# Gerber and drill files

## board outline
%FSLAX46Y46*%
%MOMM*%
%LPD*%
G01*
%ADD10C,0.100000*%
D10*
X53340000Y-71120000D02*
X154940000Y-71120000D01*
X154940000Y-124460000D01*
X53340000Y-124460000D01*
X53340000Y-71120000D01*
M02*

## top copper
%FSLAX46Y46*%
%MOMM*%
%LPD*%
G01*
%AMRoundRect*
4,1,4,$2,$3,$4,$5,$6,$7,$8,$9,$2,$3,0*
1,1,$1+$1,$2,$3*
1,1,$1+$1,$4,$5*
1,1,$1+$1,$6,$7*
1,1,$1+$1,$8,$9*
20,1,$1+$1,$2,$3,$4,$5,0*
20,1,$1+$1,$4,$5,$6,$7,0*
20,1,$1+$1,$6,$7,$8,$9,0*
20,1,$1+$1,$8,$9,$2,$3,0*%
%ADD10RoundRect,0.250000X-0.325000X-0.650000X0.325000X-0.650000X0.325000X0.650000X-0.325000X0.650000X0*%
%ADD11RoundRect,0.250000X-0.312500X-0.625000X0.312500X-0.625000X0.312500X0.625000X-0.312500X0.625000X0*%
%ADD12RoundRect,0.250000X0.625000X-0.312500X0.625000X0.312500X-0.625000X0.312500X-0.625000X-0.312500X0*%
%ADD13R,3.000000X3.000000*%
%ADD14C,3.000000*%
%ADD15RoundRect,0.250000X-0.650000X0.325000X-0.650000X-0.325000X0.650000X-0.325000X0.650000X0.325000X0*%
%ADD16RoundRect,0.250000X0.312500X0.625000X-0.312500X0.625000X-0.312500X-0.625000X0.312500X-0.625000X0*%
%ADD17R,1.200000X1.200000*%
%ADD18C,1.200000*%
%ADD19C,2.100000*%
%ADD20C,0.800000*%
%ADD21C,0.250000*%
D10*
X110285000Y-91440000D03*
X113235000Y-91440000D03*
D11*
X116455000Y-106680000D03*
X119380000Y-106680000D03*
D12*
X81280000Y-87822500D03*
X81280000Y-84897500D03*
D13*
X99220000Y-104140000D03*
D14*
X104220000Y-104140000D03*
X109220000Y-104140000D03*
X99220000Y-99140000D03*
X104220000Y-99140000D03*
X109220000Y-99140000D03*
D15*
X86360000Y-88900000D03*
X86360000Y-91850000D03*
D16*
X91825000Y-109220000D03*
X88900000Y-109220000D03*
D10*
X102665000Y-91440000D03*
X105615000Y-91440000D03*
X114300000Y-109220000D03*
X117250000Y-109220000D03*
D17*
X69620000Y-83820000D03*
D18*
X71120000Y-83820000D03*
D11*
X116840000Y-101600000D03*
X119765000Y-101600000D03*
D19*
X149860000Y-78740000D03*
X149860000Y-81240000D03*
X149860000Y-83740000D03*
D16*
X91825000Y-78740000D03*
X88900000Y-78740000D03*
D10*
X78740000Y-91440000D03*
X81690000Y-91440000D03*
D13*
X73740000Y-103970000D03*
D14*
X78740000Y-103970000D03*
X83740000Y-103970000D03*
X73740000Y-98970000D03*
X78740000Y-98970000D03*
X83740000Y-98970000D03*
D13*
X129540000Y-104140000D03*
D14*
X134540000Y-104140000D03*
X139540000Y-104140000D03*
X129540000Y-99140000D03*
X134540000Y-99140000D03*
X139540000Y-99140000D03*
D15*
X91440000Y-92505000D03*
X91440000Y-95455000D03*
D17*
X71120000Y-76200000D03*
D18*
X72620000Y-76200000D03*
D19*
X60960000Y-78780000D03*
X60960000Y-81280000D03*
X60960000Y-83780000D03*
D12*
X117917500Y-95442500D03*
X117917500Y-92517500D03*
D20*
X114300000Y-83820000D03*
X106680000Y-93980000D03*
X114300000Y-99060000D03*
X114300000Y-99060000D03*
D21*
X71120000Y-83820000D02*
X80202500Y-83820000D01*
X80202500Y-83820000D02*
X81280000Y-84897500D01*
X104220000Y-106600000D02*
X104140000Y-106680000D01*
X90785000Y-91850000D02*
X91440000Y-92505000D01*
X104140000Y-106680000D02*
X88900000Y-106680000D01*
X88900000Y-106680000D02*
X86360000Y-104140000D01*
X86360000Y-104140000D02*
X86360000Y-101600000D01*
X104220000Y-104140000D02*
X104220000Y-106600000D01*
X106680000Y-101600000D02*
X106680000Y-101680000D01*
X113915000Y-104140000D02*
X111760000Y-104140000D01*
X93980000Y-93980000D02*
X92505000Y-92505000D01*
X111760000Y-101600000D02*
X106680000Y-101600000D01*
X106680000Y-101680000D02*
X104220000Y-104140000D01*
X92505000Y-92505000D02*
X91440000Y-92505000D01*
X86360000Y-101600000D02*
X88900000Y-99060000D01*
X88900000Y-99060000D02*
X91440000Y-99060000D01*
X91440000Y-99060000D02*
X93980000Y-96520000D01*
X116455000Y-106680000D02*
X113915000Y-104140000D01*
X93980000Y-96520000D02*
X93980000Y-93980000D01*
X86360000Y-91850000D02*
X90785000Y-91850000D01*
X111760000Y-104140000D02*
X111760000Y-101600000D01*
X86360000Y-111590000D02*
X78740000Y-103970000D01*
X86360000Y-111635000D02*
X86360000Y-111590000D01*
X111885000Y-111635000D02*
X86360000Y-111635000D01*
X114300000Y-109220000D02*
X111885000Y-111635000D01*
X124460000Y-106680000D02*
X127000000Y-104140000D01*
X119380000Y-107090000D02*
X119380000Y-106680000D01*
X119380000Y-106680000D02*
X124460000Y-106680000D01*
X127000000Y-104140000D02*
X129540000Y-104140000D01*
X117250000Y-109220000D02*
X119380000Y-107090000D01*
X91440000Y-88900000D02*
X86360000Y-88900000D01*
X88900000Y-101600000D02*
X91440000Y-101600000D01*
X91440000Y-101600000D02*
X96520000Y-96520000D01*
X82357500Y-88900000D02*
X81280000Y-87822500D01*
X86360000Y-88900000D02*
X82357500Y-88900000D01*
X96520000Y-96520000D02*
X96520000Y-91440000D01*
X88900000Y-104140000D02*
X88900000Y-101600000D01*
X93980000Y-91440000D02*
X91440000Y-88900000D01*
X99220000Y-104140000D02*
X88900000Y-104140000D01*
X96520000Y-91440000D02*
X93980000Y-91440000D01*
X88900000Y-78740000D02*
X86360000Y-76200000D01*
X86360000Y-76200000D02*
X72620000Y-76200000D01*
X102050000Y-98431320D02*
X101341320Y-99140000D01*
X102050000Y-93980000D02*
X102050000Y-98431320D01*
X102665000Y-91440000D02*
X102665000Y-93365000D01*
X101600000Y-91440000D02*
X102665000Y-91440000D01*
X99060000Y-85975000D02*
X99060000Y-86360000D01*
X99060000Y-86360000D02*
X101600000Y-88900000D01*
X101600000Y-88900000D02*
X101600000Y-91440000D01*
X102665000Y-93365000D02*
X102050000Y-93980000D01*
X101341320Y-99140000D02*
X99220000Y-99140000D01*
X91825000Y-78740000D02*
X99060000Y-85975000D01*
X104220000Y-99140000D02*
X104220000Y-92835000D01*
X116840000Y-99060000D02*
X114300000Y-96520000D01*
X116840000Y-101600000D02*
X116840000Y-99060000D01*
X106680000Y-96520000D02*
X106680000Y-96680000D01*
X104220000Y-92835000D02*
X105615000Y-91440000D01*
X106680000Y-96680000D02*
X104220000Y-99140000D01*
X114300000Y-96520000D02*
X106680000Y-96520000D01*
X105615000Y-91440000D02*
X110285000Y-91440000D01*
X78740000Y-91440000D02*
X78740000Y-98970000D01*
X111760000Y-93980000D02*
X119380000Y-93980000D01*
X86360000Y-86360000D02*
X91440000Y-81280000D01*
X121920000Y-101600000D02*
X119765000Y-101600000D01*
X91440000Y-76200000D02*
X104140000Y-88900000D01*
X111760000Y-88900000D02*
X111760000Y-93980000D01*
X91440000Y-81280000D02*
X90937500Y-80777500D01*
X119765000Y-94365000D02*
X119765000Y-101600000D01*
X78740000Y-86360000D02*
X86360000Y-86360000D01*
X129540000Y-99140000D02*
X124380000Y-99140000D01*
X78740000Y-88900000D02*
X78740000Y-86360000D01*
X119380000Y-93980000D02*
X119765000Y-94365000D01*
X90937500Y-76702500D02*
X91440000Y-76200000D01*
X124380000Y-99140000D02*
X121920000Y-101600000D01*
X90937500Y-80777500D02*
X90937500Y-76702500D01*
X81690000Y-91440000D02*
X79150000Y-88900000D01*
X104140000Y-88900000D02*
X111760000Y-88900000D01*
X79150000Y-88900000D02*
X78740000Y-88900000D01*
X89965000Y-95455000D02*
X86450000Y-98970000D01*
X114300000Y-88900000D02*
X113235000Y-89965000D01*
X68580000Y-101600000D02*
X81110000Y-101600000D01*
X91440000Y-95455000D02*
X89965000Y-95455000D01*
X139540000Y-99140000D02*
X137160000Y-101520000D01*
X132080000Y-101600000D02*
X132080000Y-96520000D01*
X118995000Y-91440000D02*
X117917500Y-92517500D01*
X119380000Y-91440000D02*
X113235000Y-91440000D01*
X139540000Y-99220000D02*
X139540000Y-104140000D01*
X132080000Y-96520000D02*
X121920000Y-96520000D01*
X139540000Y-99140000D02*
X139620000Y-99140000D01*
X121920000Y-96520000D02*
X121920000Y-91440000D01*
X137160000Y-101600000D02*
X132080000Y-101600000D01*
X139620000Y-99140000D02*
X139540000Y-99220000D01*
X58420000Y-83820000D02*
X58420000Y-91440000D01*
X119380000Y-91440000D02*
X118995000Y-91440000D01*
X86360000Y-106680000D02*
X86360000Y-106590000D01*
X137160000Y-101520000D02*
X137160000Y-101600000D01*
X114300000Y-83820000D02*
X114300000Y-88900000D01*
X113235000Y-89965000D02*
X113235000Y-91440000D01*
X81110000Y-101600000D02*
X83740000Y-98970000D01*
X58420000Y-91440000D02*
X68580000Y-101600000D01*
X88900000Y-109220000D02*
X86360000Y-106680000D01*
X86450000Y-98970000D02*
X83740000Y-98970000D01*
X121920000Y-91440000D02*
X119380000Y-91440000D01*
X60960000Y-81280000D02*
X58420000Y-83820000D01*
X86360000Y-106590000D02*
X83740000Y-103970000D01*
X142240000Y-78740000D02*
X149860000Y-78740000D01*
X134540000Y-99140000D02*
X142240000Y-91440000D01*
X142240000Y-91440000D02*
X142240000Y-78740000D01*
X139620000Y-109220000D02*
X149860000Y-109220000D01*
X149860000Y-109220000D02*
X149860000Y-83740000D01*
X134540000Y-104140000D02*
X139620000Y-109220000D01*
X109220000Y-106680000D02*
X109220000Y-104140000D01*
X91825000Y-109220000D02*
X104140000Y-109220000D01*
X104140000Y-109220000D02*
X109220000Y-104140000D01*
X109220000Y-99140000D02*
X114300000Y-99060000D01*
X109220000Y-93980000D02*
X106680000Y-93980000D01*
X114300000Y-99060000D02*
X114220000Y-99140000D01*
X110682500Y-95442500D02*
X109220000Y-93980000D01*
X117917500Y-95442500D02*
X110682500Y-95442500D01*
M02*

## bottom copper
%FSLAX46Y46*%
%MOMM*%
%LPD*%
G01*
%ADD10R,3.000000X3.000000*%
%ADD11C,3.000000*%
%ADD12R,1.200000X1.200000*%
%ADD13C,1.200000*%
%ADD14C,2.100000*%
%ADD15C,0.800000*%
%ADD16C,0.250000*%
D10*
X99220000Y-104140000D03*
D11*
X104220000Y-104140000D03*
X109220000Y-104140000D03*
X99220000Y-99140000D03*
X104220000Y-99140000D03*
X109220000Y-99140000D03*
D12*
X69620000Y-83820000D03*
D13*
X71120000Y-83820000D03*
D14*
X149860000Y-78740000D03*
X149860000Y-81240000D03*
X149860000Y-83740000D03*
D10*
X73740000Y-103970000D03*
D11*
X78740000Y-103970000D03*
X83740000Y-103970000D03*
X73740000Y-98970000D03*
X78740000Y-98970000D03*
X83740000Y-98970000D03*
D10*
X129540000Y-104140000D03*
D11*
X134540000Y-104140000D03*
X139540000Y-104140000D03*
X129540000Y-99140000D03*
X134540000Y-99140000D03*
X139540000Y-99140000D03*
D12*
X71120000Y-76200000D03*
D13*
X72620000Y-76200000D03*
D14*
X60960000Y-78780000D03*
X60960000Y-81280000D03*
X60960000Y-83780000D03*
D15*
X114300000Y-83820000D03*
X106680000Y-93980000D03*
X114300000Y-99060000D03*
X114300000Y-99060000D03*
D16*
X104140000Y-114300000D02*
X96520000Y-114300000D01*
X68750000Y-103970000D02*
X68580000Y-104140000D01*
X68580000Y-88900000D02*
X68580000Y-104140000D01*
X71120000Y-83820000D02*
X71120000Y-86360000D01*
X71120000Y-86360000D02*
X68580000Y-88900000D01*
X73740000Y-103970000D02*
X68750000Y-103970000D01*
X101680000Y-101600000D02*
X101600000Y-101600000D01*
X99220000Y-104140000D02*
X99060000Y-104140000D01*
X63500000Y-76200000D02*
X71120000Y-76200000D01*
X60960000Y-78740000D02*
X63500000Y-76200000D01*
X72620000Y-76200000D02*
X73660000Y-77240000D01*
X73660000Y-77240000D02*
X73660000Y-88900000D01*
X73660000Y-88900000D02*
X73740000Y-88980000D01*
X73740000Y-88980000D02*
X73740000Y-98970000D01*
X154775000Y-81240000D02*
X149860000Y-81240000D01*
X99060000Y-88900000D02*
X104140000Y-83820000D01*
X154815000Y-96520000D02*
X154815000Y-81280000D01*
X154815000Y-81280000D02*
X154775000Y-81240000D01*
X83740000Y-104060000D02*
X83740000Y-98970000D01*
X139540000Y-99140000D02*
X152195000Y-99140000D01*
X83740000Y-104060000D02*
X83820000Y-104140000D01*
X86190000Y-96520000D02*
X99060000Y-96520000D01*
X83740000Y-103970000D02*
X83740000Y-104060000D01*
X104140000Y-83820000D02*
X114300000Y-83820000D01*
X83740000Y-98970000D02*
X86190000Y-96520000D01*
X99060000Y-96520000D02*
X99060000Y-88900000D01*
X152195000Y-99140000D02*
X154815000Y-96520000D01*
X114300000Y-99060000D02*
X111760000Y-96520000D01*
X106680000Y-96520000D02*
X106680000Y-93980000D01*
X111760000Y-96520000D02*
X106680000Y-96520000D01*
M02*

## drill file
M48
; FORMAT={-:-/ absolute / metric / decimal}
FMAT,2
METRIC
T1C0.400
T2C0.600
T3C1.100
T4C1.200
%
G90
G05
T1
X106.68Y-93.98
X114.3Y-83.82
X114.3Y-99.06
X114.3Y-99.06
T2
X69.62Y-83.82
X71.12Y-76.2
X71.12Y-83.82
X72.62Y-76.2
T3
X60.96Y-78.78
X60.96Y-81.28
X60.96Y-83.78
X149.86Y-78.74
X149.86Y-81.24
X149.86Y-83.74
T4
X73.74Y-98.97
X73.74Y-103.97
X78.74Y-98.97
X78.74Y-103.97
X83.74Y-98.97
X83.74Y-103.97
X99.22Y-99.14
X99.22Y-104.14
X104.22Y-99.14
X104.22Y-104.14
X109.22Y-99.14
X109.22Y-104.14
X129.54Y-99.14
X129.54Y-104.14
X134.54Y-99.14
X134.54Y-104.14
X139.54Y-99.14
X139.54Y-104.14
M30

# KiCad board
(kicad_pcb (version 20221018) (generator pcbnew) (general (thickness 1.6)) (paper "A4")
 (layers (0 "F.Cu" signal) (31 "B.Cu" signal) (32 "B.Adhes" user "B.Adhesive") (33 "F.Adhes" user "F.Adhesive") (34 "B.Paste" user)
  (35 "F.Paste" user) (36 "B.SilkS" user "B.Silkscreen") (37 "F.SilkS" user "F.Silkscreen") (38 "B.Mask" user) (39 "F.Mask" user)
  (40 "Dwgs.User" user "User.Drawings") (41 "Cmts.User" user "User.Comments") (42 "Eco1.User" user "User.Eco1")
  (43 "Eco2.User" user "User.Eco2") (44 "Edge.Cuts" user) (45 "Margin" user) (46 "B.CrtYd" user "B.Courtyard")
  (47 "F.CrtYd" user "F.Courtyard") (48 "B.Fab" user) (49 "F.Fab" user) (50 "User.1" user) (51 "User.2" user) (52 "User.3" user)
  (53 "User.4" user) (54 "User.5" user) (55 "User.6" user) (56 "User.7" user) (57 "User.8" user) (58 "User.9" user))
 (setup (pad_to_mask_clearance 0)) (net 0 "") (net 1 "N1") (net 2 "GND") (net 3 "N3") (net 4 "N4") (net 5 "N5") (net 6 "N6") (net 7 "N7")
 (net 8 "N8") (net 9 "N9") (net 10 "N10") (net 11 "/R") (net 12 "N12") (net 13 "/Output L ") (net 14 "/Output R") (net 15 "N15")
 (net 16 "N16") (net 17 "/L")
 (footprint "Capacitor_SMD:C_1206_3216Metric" (layer "F.Cu") (at 111.76 91.44)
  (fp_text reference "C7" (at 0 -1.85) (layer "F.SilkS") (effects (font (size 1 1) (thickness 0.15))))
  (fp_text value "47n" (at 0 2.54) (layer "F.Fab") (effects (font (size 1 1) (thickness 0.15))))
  (pad "1" smd roundrect (at -1.475 0) (size 1.15 1.8) (layers "F.Cu" "F.Paste" "F.Mask") (roundrect_rratio 0.217391) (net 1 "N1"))
  (pad "2" smd roundrect (at 1.475 0) (size 1.15 1.8) (layers "F.Cu" "F.Paste" "F.Mask") (roundrect_rratio 0.217391) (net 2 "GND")))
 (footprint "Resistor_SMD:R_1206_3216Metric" (layer "F.Cu") (at 117.9175 106.68)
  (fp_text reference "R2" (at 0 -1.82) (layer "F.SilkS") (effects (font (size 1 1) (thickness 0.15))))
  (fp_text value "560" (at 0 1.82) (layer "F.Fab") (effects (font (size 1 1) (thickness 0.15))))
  (pad "1" smd roundrect (at -1.4625 0) (size 1.125 1.75) (layers "F.Cu" "F.Paste" "F.Mask") (roundrect_rratio 0.222222) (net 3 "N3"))
  (pad "2" smd roundrect (at 1.4625 0) (size 1.125 1.75) (layers "F.Cu" "F.Paste" "F.Mask") (roundrect_rratio 0.222222) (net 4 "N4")))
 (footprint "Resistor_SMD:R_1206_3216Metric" (layer "F.Cu") (at 81.28 86.36 90)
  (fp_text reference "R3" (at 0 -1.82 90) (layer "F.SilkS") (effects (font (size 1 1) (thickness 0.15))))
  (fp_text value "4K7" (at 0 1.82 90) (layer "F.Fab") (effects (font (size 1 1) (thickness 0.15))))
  (pad "1" smd roundrect (at -1.4625 0 90) (size 1.125 1.75) (layers "F.Cu" "F.Paste" "F.Mask") (roundrect_rratio 0.222222) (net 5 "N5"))
  (pad "2" smd roundrect (at 1.4625 0 90) (size 1.125 1.75) (layers "F.Cu" "F.Paste" "F.Mask") (roundrect_rratio 0.222222) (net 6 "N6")))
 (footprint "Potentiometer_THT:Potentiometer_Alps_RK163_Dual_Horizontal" (layer "F.Cu") (at 99.22 104.14 90)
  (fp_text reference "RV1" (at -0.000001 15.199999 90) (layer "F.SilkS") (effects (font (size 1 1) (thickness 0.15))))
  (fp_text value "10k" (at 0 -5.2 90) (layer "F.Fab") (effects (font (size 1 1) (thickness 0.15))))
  (pad "1" thru_hole rect (at 0 0 270) (size 3 3) (drill 1.2) (layers "*.Cu" "*.Mask") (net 5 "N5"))
  (pad "2" thru_hole circle (at 0 5 270) (size 3 3) (drill 1.2) (layers "*.Cu" "*.Mask") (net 3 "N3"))
  (pad "3" thru_hole circle (at 0 10 270) (size 3 3) (drill 1.2) (layers "*.Cu" "*.Mask") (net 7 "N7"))
  (pad "4" thru_hole circle (at 5 0 270) (size 3 3) (drill 1.2) (layers "*.Cu" "*.Mask") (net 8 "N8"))
  (pad "5" thru_hole circle (at 5 5 270) (size 3 3) (drill 1.2) (layers "*.Cu" "*.Mask") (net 1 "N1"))
  (pad "6" thru_hole circle (at 5 10 270) (size 3 3) (drill 1.2) (layers "*.Cu" "*.Mask") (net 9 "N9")))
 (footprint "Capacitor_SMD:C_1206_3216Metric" (layer "F.Cu") (at 86.36 90.375 -90)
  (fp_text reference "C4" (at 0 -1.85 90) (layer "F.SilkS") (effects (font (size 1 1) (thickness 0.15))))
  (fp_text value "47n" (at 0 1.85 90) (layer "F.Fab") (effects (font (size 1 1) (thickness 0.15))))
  (pad "1" smd roundrect (at -1.475 0 270) (size 1.15 1.8) (layers "F.Cu" "F.Paste" "F.Mask") (roundrect_rratio 0.217391) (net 5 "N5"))
  (pad "2" smd roundrect (at 1.475 0 270) (size 1.15 1.8) (layers "F.Cu" "F.Paste" "F.Mask") (roundrect_rratio 0.217391) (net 3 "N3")))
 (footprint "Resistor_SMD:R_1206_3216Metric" (layer "F.Cu") (at 90.3625 109.22 180)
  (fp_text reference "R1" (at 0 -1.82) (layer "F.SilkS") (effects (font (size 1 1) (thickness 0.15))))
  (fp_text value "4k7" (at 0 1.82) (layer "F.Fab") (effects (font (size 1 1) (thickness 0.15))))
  (pad "1" smd roundrect (at -1.4625 0 180) (size 1.125 1.75) (layers "F.Cu" "F.Paste" "F.Mask") (roundrect_rratio 0.222222) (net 7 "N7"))
  (pad "2" smd roundrect (at 1.4625 0 180) (size 1.125 1.75) (layers "F.Cu" "F.Paste" "F.Mask") (roundrect_rratio 0.222222) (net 2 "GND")))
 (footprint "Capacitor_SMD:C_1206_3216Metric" (layer "F.Cu") (at 104.14 91.44)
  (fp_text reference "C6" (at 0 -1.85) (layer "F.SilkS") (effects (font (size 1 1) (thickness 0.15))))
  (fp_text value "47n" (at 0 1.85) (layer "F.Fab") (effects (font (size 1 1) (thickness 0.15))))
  (pad "1" smd roundrect (at -1.475 0) (size 1.15 1.8) (layers "F.Cu" "F.Paste" "F.Mask") (roundrect_rratio 0.217391) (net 8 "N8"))
  (pad "2" smd roundrect (at 1.475 0) (size 1.15 1.8) (layers "F.Cu" "F.Paste" "F.Mask") (roundrect_rratio 0.217391) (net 1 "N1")))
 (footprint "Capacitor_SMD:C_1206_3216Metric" (layer "F.Cu") (at 115.775 109.22)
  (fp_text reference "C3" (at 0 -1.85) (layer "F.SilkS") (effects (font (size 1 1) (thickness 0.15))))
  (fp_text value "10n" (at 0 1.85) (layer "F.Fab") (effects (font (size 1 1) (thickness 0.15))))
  (pad "1" smd roundrect (at -1.475 0) (size 1.15 1.8) (layers "F.Cu" "F.Paste" "F.Mask") (roundrect_rratio 0.217391) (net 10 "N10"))
  (pad "2" smd roundrect (at 1.475 0) (size 1.15 1.8) (layers "F.Cu" "F.Paste" "F.Mask") (roundrect_rratio 0.217391) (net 4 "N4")))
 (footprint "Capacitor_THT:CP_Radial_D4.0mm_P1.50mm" (layer "F.Cu") (at 69.62 83.82)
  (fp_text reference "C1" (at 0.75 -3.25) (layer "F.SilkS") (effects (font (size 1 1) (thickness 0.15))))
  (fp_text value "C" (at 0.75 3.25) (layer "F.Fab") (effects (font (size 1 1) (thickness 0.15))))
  (pad "1" thru_hole rect (at 0 0) (size 1.2 1.2) (drill 0.6) (layers "*.Cu" "*.Mask") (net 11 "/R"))
  (pad "2" thru_hole circle (at 1.5 0) (size 1.2 1.2) (drill 0.6) (layers "*.Cu" "*.Mask") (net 6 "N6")))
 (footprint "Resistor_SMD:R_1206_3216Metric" (layer "F.Cu") (at 118.3025 101.6)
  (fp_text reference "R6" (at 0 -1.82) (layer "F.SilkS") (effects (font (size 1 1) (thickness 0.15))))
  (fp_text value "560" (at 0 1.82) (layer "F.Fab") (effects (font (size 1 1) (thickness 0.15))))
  (pad "1" smd roundrect (at -1.4625 0) (size 1.125 1.75) (layers "F.Cu" "F.Paste" "F.Mask") (roundrect_rratio 0.222222) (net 1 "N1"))
  (pad "2" smd roundrect (at 1.4625 0) (size 1.125 1.75) (layers "F.Cu" "F.Paste" "F.Mask") (roundrect_rratio 0.222222) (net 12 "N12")))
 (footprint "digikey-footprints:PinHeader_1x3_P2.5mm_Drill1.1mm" (layer "F.Cu") (at 149.86 78.74 -90)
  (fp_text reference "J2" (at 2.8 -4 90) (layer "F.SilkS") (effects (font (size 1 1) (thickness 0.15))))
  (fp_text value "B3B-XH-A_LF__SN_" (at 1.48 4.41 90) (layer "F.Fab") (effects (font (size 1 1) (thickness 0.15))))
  (pad "1" thru_hole circle (at 0 0 270) (size 2.1 2.1) (drill 1.1) (layers "*.Cu" "*.Mask") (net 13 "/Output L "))
  (pad "2" thru_hole circle (at 2.5 0 270) (size 2.1 2.1) (drill 1.1) (layers "*.Cu" "*.Mask") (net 2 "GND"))
  (pad "3" thru_hole circle (at 5 0 270) (size 2.1 2.1) (drill 1.1) (layers "*.Cu" "*.Mask") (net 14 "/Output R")))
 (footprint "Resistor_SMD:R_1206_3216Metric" (layer "F.Cu") (at 90.3625 78.74 180)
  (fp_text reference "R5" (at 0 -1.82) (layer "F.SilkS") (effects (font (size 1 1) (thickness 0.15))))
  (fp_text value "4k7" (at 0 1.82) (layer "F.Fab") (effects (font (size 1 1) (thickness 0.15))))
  (pad "1" smd roundrect (at -1.4625 0 180) (size 1.125 1.75) (layers "F.Cu" "F.Paste" "F.Mask") (roundrect_rratio 0.222222) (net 8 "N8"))
  (pad "2" smd roundrect (at 1.4625 0 180) (size 1.125 1.75) (layers "F.Cu" "F.Paste" "F.Mask") (roundrect_rratio 0.222222) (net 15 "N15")))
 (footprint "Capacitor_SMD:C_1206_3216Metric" (layer "F.Cu") (at 80.215 91.44)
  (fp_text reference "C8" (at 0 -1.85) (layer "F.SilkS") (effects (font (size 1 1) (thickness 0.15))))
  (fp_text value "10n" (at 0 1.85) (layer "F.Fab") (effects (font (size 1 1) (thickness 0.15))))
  (pad "1" smd roundrect (at -1.475 0) (size 1.15 1.8) (layers "F.Cu" "F.Paste" "F.Mask") (roundrect_rratio 0.217391) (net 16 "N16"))
  (pad "2" smd roundrect (at 1.475 0) (size 1.15 1.8) (layers "F.Cu" "F.Paste" "F.Mask") (roundrect_rratio 0.217391) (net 12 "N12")))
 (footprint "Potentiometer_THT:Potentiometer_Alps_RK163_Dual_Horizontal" (layer "F.Cu") (at 73.74 103.97 90)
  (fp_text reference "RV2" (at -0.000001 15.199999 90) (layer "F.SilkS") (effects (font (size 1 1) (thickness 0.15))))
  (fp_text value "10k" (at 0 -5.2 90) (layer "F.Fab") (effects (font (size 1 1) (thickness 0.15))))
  (pad "1" thru_hole rect (at 0 0 270) (size 3 3) (drill 1.2) (layers "*.Cu" "*.Mask") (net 6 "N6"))
  (pad "2" thru_hole circle (at 0 5 270) (size 3 3) (drill 1.2) (layers "*.Cu" "*.Mask") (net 10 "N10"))
  (pad "3" thru_hole circle (at 0 10 270) (size 3 3) (drill 1.2) (layers "*.Cu" "*.Mask") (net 2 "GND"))
  (pad "4" thru_hole circle (at 5 0 270) (size 3 3) (drill 1.2) (layers "*.Cu" "*.Mask") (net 15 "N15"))
  (pad "5" thru_hole circle (at 5 5 270) (size 3 3) (drill 1.2) (layers "*.Cu" "*.Mask") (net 16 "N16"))
  (pad "6" thru_hole circle (at 5 10 270) (size 3 3) (drill 1.2) (layers "*.Cu" "*.Mask") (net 2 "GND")))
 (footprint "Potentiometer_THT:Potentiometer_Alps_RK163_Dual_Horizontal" (layer "F.Cu") (at 129.54 104.14 90)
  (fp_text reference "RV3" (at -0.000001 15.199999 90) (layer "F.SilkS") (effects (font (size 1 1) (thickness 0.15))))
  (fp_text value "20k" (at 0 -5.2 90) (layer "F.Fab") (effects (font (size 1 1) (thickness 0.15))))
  (pad "1" thru_hole rect (at 0 0 270) (size 3 3) (drill 1.2) (layers "*.Cu" "*.Mask") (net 4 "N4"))
  (pad "2" thru_hole circle (at 0 5 270) (size 3 3) (drill 1.2) (layers "*.Cu" "*.Mask") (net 14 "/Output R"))
  (pad "3" thru_hole circle (at 0 10 270) (size 3 3) (drill 1.2) (layers "*.Cu" "*.Mask") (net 2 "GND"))
  (pad "4" thru_hole circle (at 5 0 270) (size 3 3) (drill 1.2) (layers "*.Cu" "*.Mask") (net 12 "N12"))
  (pad "5" thru_hole circle (at 5 5 270) (size 3 3) (drill 1.2) (layers "*.Cu" "*.Mask") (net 13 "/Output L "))
  (pad "6" thru_hole circle (at 5 10 270) (size 3 3) (drill 1.2) (layers "*.Cu" "*.Mask") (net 2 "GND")))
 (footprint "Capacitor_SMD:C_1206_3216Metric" (layer "F.Cu") (at 91.44 93.98 -90)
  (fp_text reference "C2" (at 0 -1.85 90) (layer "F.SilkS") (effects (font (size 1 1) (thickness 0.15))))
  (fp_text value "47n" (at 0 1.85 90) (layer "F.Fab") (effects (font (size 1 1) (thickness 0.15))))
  (pad "1" smd roundrect (at -1.475 0 270) (size 1.15 1.8) (layers "F.Cu" "F.Paste" "F.Mask") (roundrect_rratio 0.217391) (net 3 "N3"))
  (pad "2" smd roundrect (at 1.475 0 270) (size 1.15 1.8) (layers "F.Cu" "F.Paste" "F.Mask") (roundrect_rratio 0.217391) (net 2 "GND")))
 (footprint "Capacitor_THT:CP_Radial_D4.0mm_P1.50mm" (layer "F.Cu") (at 71.12 76.2)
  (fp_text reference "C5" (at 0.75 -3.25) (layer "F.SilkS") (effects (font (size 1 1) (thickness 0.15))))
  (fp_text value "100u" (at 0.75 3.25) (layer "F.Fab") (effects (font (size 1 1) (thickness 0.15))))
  (pad "1" thru_hole rect (at 0 0) (size 1.2 1.2) (drill 0.6) (layers "*.Cu" "*.Mask") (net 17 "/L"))
  (pad "2" thru_hole circle (at 1.5 0) (size 1.2 1.2) (drill 0.6) (layers "*.Cu" "*.Mask") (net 15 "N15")))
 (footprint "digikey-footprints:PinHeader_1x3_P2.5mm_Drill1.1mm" (layer "F.Cu") (at 60.96 78.78 -90)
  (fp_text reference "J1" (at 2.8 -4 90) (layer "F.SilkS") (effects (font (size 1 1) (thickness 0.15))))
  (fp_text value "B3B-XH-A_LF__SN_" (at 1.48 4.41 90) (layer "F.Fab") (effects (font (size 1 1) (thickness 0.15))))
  (pad "1" thru_hole circle (at 0 0 270) (size 2.1 2.1) (drill 1.1) (layers "*.Cu" "*.Mask") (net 17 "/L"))
  (pad "2" thru_hole circle (at 2.5 0 270) (size 2.1 2.1) (drill 1.1) (layers "*.Cu" "*.Mask") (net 2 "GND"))
  (pad "3" thru_hole circle (at 5 0 270) (size 2.1 2.1) (drill 1.1) (layers "*.Cu" "*.Mask") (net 11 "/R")))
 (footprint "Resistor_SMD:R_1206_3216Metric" (layer "F.Cu") (at 117.9175 93.98 90)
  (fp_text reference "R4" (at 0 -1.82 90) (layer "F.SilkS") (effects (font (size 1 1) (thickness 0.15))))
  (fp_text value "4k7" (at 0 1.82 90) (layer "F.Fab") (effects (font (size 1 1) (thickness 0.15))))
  (pad "1" smd roundrect (at -1.4625 0 90) (size 1.125 1.75) (layers "F.Cu" "F.Paste" "F.Mask") (roundrect_rratio 0.222222) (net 9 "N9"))
  (pad "2" smd roundrect (at 1.4625 0 90) (size 1.125 1.75) (layers "F.Cu" "F.Paste" "F.Mask") (roundrect_rratio 0.222222) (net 2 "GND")))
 (gr_rect (start 53.34 71.12) (end 154.94 124.46) (stroke (width 0.1) (type default)) (fill none) (layer "Edge.Cuts"))
 (segment (start 104.14 114.3) (end 96.52 114.3) (width 0.25) (layer "B.Cu") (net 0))
 (segment (start 71.12 83.82) (end 80.2025 83.82) (width 0.25) (layer "F.Cu") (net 6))
 (segment (start 80.2025 83.82) (end 81.28 84.8975) (width 0.25) (layer "F.Cu") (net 6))
 (segment (start 68.75 103.97) (end 68.58 104.14) (width 0.25) (layer "B.Cu") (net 6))
 (segment (start 68.58 88.9) (end 68.58 104.14) (width 0.25) (layer "B.Cu") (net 6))
 (segment (start 71.12 83.82) (end 71.12 86.36) (width 0.25) (layer "B.Cu") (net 6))
 (segment (start 71.12 86.36) (end 68.58 88.9) (width 0.25) (layer "B.Cu") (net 6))
 (segment (start 73.74 103.97) (end 68.75 103.97) (width 0.25) (layer "B.Cu") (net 6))
 (segment (start 104.22 106.6) (end 104.14 106.68) (width 0.25) (layer "F.Cu") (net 3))
 (segment (start 90.785 91.85) (end 91.44 92.505) (width 0.25) (layer "F.Cu") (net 3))
 (segment (start 104.14 106.68) (end 88.9 106.68) (width 0.25) (layer "F.Cu") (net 3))
 (segment (start 88.9 106.68) (end 86.36 104.14) (width 0.25) (layer "F.Cu") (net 3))
 (segment (start 86.36 104.14) (end 86.36 101.6) (width 0.25) (layer "F.Cu") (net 3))
 (segment (start 104.22 104.14) (end 104.22 106.6) (width 0.25) (layer "F.Cu") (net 3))
 (segment (start 106.68 101.6) (end 106.68 101.68) (width 0.25) (layer "F.Cu") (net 3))
 (segment (start 113.915 104.14) (end 111.76 104.14) (width 0.25) (layer "F.Cu") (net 3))
 (segment (start 93.98 93.98) (end 92.505 92.505) (width 0.25) (layer "F.Cu") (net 3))
 (segment (start 111.76 101.6) (end 106.68 101.6) (width 0.25) (layer "F.Cu") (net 3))
 (segment (start 106.68 101.68) (end 104.22 104.14) (width 0.25) (layer "F.Cu") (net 3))
 (segment (start 92.505 92.505) (end 91.44 92.505) (width 0.25) (layer "F.Cu") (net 3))
 (segment (start 86.36 101.6) (end 88.9 99.06) (width 0.25) (layer "F.Cu") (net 3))
 (segment (start 88.9 99.06) (end 91.44 99.06) (width 0.25) (layer "F.Cu") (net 3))
 (segment (start 91.44 99.06) (end 93.98 96.52) (width 0.25) (layer "F.Cu") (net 3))
 (segment (start 116.455 106.68) (end 113.915 104.14) (width 0.25) (layer "F.Cu") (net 3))
 (segment (start 93.98 96.52) (end 93.98 93.98) (width 0.25) (layer "F.Cu") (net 3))
 (segment (start 86.36 91.85) (end 90.785 91.85) (width 0.25) (layer "F.Cu") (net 3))
 (segment (start 111.76 104.14) (end 111.76 101.6) (width 0.25) (layer "F.Cu") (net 3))
 (segment (start 101.68 101.6) (end 101.6 101.6) (width 0.25) (layer "B.Cu") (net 3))
 (segment (start 86.36 111.59) (end 78.74 103.97) (width 0.25) (layer "F.Cu") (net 10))
 (segment (start 86.36 111.635) (end 86.36 111.59) (width 0.25) (layer "F.Cu") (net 10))
 (segment (start 111.885 111.635) (end 86.36 111.635) (width 0.25) (layer "F.Cu") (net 10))
 (segment (start 114.3 109.22) (end 111.885 111.635) (width 0.25) (layer "F.Cu") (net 10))
 (segment (start 124.46 106.68) (end 127 104.14) (width 0.25) (layer "F.Cu") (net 4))
 (segment (start 119.38 107.09) (end 119.38 106.68) (width 0.25) (layer "F.Cu") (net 4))
 (segment (start 119.38 106.68) (end 124.46 106.68) (width 0.25) (layer "F.Cu") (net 4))
 (segment (start 127 104.14) (end 129.54 104.14) (width 0.25) (layer "F.Cu") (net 4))
 (segment (start 117.25 109.22) (end 119.38 107.09) (width 0.25) (layer "F.Cu") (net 4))
 (segment (start 91.44 88.9) (end 86.36 88.9) (width 0.25) (layer "F.Cu") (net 5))
 (segment (start 88.9 101.6) (end 91.44 101.6) (width 0.25) (layer "F.Cu") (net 5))
 (segment (start 91.44 101.6) (end 96.52 96.52) (width 0.25) (layer "F.Cu") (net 5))
 (segment (start 82.3575 88.9) (end 81.28 87.8225) (width 0.25) (layer "F.Cu") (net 5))
 (segment (start 86.36 88.9) (end 82.3575 88.9) (width 0.25) (layer "F.Cu") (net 5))
 (segment (start 96.52 96.52) (end 96.52 91.44) (width 0.25) (layer "F.Cu") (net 5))
 (segment (start 88.9 104.14) (end 88.9 101.6) (width 0.25) (layer "F.Cu") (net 5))
 (segment (start 93.98 91.44) (end 91.44 88.9) (width 0.25) (layer "F.Cu") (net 5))
 (segment (start 99.22 104.14) (end 88.9 104.14) (width 0.25) (layer "F.Cu") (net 5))
 (segment (start 96.52 91.44) (end 93.98 91.44) (width 0.25) (layer "F.Cu") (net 5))
 (segment (start 99.22 104.14) (end 99.06 104.14) (width 0.25) (layer "B.Cu") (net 5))
 (segment (start 63.5 76.2) (end 71.12 76.2) (width 0.25) (layer "B.Cu") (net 17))
 (segment (start 60.96 78.74) (end 63.5 76.2) (width 0.25) (layer "B.Cu") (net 17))
 (segment (start 88.9 78.74) (end 86.36 76.2) (width 0.25) (layer "F.Cu") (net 15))
 (segment (start 86.36 76.2) (end 72.62 76.2) (width 0.25) (layer "F.Cu") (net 15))
 (segment (start 72.62 76.2) (end 73.66 77.24) (width 0.25) (layer "B.Cu") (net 15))
 (segment (start 73.66 77.24) (end 73.66 88.9) (width 0.25) (layer "B.Cu") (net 15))
 (segment (start 73.66 88.9) (end 73.74 88.98) (width 0.25) (layer "B.Cu") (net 15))
 (segment (start 73.74 88.98) (end 73.74 98.97) (width 0.25) (layer "B.Cu") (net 15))
 (segment (start 102.05 98.43132) (end 101.34132 99.14) (width 0.25) (layer "F.Cu") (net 8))
 (segment (start 102.05 93.98) (end 102.05 98.43132) (width 0.25) (layer "F.Cu") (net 8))
 (segment (start 102.665 91.44) (end 102.665 93.365) (width 0.25) (layer "F.Cu") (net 8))
 (segment (start 101.6 91.44) (end 102.665 91.44) (width 0.25) (layer "F.Cu") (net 8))
 (segment (start 99.06 85.975) (end 99.06 86.36) (width 0.25) (layer "F.Cu") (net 8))
 (segment (start 99.06 86.36) (end 101.6 88.9) (width 0.25) (layer "F.Cu") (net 8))
 (segment (start 101.6 88.9) (end 101.6 91.44) (width 0.25) (layer "F.Cu") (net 8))
 (segment (start 102.665 93.365) (end 102.05 93.98) (width 0.25) (layer "F.Cu") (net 8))
 (segment (start 101.34132 99.14) (end 99.22 99.14) (width 0.25) (layer "F.Cu") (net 8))
 (segment (start 91.825 78.74) (end 99.06 85.975) (width 0.25) (layer "F.Cu") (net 8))
 (segment (start 104.22 99.14) (end 104.22 92.835) (width 0.25) (layer "F.Cu") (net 1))
 (segment (start 116.84 99.06) (end 114.3 96.52) (width 0.25) (layer "F.Cu") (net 1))
 (segment (start 116.84 101.6) (end 116.84 99.06) (width 0.25) (layer "F.Cu") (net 1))
 (segment (start 106.68 96.52) (end 106.68 96.68) (width 0.25) (layer "F.Cu") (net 1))
 (segment (start 104.22 92.835) (end 105.615 91.44) (width 0.25) (layer "F.Cu") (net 1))
 (segment (start 106.68 96.68) (end 104.22 99.14) (width 0.25) (layer "F.Cu") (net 1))
 (segment (start 114.3 96.52) (end 106.68 96.52) (width 0.25) (layer "F.Cu") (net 1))
 (segment (start 105.615 91.44) (end 110.285 91.44) (width 0.25) (layer "F.Cu") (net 1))
 (segment (start 78.74 91.44) (end 78.74 98.97) (width 0.25) (layer "F.Cu") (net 16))
 (segment (start 111.76 93.98) (end 119.38 93.98) (width 0.25) (layer "F.Cu") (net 12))
 (segment (start 86.36 86.36) (end 91.44 81.28) (width 0.25) (layer "F.Cu") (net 12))
 (segment (start 121.92 101.6) (end 119.765 101.6) (width 0.25) (layer "F.Cu") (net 12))
 (segment (start 91.44 76.2) (end 104.14 88.9) (width 0.25) (layer "F.Cu") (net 12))
 (segment (start 111.76 88.9) (end 111.76 93.98) (width 0.25) (layer "F.Cu") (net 12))
 (segment (start 91.44 81.28) (end 90.9375 80.7775) (width 0.25) (layer "F.Cu") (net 12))
 (segment (start 119.765 94.365) (end 119.765 101.6) (width 0.25) (layer "F.Cu") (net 12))
 (segment (start 78.74 86.36) (end 86.36 86.36) (width 0.25) (layer "F.Cu") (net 12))
 (segment (start 129.54 99.14) (end 124.38 99.14) (width 0.25) (layer "F.Cu") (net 12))
 (segment (start 78.74 88.9) (end 78.74 86.36) (width 0.25) (layer "F.Cu") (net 12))
 (segment (start 119.38 93.98) (end 119.765 94.365) (width 0.25) (layer "F.Cu") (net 12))
 (segment (start 90.9375 76.7025) (end 91.44 76.2) (width 0.25) (layer "F.Cu") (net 12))
 (segment (start 124.38 99.14) (end 121.92 101.6) (width 0.25) (layer "F.Cu") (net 12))
 (segment (start 90.9375 80.7775) (end 90.9375 76.7025) (width 0.25) (layer "F.Cu") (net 12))
 (segment (start 81.69 91.44) (end 79.15 88.9) (width 0.25) (layer "F.Cu") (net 12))
 (segment (start 104.14 88.9) (end 111.76 88.9) (width 0.25) (layer "F.Cu") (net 12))
 (segment (start 79.15 88.9) (end 78.74 88.9) (width 0.25) (layer "F.Cu") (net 12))
 (segment (start 89.965 95.455) (end 86.45 98.97) (width 0.25) (layer "F.Cu") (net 2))
 (segment (start 114.3 88.9) (end 113.235 89.965) (width 0.25) (layer "F.Cu") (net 2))
 (segment (start 68.58 101.6) (end 81.11 101.6) (width 0.25) (layer "F.Cu") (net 2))
 (segment (start 91.44 95.455) (end 89.965 95.455) (width 0.25) (layer "F.Cu") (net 2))
 (segment (start 139.54 99.14) (end 137.16 101.52) (width 0.25) (layer "F.Cu") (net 2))
 (segment (start 132.08 101.6) (end 132.08 96.52) (width 0.25) (layer "F.Cu") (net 2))
 (segment (start 118.995 91.44) (end 117.9175 92.5175) (width 0.25) (layer "F.Cu") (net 2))
 (segment (start 119.38 91.44) (end 113.235 91.44) (width 0.25) (layer "F.Cu") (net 2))
 (segment (start 139.54 99.22) (end 139.54 104.14) (width 0.25) (layer "F.Cu") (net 2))
 (segment (start 132.08 96.52) (end 121.92 96.52) (width 0.25) (layer "F.Cu") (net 2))
 (segment (start 139.54 99.14) (end 139.62 99.14) (width 0.25) (layer "F.Cu") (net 2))
 (segment (start 121.92 96.52) (end 121.92 91.44) (width 0.25) (layer "F.Cu") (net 2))
 (segment (start 137.16 101.6) (end 132.08 101.6) (width 0.25) (layer "F.Cu") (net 2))
 (segment (start 139.62 99.14) (end 139.54 99.22) (width 0.25) (layer "F.Cu") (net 2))
 (segment (start 58.42 83.82) (end 58.42 91.44) (width 0.25) (layer "F.Cu") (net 2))
 (segment (start 119.38 91.44) (end 118.995 91.44) (width 0.25) (layer "F.Cu") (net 2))
 (segment (start 86.36 106.68) (end 86.36 106.59) (width 0.25) (layer "F.Cu") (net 2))
 (segment (start 137.16 101.52) (end 137.16 101.6) (width 0.25) (layer "F.Cu") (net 2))
 (segment (start 114.3 83.82) (end 114.3 88.9) (width 0.25) (layer "F.Cu") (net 2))
 (segment (start 113.235 89.965) (end 113.235 91.44) (width 0.25) (layer "F.Cu") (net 2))
 (segment (start 81.11 101.6) (end 83.74 98.97) (width 0.25) (layer "F.Cu") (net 2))
 (segment (start 58.42 91.44) (end 68.58 101.6) (width 0.25) (layer "F.Cu") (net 2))
 (segment (start 88.9 109.22) (end 86.36 106.68) (width 0.25) (layer "F.Cu") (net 2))
 (segment (start 86.45 98.97) (end 83.74 98.97) (width 0.25) (layer "F.Cu") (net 2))
 (segment (start 121.92 91.44) (end 119.38 91.44) (width 0.25) (layer "F.Cu") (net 2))
 (segment (start 60.96 81.28) (end 58.42 83.82) (width 0.25) (layer "F.Cu") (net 2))
 (segment (start 86.36 106.59) (end 83.74 103.97) (width 0.25) (layer "F.Cu") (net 2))
 (via (at 114.3 83.82) (size 0.8) (drill 0.4) (layers "F.Cu" "B.Cu") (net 2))
 (segment (start 154.775 81.24) (end 149.86 81.24) (width 0.25) (layer "B.Cu") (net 2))
 (segment (start 99.06 88.9) (end 104.14 83.82) (width 0.25) (layer "B.Cu") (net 2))
 (segment (start 154.815 96.52) (end 154.815 81.28) (width 0.25) (layer "B.Cu") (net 2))
 (segment (start 154.815 81.28) (end 154.775 81.24) (width 0.25) (layer "B.Cu") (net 2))
 (segment (start 83.74 104.06) (end 83.74 98.97) (width 0.25) (layer "B.Cu") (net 2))
 (segment (start 139.54 99.14) (end 152.195 99.14) (width 0.25) (layer "B.Cu") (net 2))
 (segment (start 83.74 104.06) (end 83.82 104.14) (width 0.25) (layer "B.Cu") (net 2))
 (segment (start 86.19 96.52) (end 99.06 96.52) (width 0.25) (layer "B.Cu") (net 2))
 (segment (start 83.74 103.97) (end 83.74 104.06) (width 0.25) (layer "B.Cu") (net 2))
 (segment (start 104.14 83.82) (end 114.3 83.82) (width 0.25) (layer "B.Cu") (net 2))
 (segment (start 83.74 98.97) (end 86.19 96.52) (width 0.25) (layer "B.Cu") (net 2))
 (segment (start 99.06 96.52) (end 99.06 88.9) (width 0.25) (layer "B.Cu") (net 2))
 (segment (start 152.195 99.14) (end 154.815 96.52) (width 0.25) (layer "B.Cu") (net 2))
 (segment (start 142.24 78.74) (end 149.86 78.74) (width 0.25) (layer "F.Cu") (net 13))
 (segment (start 134.54 99.14) (end 142.24 91.44) (width 0.25) (layer "F.Cu") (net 13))
 (segment (start 142.24 91.44) (end 142.24 78.74) (width 0.25) (layer "F.Cu") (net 13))
 (segment (start 139.62 109.22) (end 149.86 109.22) (width 0.25) (layer "F.Cu") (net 14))
 (segment (start 149.86 109.22) (end 149.86 83.74) (width 0.25) (layer "F.Cu") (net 14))
 (segment (start 134.54 104.14) (end 139.62 109.22) (width 0.25) (layer "F.Cu") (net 14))
 (segment (start 109.22 106.68) (end 109.22 104.14) (width 0.25) (layer "F.Cu") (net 7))
 (segment (start 91.825 109.22) (end 104.14 109.22) (width 0.25) (layer "F.Cu") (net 7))
 (segment (start 104.14 109.22) (end 109.22 104.14) (width 0.25) (layer "F.Cu") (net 7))
 (segment (start 109.22 99.14) (end 114.3 99.06) (width 0.25) (layer "F.Cu") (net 9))
 (segment (start 109.22 93.98) (end 106.68 93.98) (width 0.25) (layer "F.Cu") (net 9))
 (segment (start 114.3 99.06) (end 114.22 99.14) (width 0.25) (layer "F.Cu") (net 9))
 (segment (start 110.6825 95.4425) (end 109.22 93.98) (width 0.25) (layer "F.Cu") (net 9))
 (segment (start 117.9175 95.4425) (end 110.6825 95.4425) (width 0.25) (layer "F.Cu") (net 9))
 (via (at 106.68 93.98) (size 0.8) (drill 0.4) (layers "F.Cu" "B.Cu") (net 9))
 (via (at 114.3 99.06) (size 0.8) (drill 0.4) (layers "F.Cu" "B.Cu") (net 9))
 (via (at 114.3 99.06) (size 0.8) (drill 0.4) (layers "F.Cu" "B.Cu") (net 9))
 (segment (start 114.3 99.06) (end 111.76 96.52) (width 0.25) (layer "B.Cu") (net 9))
 (segment (start 106.68 96.52) (end 106.68 93.98) (width 0.25) (layer "B.Cu") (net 9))
 (segment (start 111.76 96.52) (end 106.68 96.52) (width 0.25) (layer "B.Cu") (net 9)))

